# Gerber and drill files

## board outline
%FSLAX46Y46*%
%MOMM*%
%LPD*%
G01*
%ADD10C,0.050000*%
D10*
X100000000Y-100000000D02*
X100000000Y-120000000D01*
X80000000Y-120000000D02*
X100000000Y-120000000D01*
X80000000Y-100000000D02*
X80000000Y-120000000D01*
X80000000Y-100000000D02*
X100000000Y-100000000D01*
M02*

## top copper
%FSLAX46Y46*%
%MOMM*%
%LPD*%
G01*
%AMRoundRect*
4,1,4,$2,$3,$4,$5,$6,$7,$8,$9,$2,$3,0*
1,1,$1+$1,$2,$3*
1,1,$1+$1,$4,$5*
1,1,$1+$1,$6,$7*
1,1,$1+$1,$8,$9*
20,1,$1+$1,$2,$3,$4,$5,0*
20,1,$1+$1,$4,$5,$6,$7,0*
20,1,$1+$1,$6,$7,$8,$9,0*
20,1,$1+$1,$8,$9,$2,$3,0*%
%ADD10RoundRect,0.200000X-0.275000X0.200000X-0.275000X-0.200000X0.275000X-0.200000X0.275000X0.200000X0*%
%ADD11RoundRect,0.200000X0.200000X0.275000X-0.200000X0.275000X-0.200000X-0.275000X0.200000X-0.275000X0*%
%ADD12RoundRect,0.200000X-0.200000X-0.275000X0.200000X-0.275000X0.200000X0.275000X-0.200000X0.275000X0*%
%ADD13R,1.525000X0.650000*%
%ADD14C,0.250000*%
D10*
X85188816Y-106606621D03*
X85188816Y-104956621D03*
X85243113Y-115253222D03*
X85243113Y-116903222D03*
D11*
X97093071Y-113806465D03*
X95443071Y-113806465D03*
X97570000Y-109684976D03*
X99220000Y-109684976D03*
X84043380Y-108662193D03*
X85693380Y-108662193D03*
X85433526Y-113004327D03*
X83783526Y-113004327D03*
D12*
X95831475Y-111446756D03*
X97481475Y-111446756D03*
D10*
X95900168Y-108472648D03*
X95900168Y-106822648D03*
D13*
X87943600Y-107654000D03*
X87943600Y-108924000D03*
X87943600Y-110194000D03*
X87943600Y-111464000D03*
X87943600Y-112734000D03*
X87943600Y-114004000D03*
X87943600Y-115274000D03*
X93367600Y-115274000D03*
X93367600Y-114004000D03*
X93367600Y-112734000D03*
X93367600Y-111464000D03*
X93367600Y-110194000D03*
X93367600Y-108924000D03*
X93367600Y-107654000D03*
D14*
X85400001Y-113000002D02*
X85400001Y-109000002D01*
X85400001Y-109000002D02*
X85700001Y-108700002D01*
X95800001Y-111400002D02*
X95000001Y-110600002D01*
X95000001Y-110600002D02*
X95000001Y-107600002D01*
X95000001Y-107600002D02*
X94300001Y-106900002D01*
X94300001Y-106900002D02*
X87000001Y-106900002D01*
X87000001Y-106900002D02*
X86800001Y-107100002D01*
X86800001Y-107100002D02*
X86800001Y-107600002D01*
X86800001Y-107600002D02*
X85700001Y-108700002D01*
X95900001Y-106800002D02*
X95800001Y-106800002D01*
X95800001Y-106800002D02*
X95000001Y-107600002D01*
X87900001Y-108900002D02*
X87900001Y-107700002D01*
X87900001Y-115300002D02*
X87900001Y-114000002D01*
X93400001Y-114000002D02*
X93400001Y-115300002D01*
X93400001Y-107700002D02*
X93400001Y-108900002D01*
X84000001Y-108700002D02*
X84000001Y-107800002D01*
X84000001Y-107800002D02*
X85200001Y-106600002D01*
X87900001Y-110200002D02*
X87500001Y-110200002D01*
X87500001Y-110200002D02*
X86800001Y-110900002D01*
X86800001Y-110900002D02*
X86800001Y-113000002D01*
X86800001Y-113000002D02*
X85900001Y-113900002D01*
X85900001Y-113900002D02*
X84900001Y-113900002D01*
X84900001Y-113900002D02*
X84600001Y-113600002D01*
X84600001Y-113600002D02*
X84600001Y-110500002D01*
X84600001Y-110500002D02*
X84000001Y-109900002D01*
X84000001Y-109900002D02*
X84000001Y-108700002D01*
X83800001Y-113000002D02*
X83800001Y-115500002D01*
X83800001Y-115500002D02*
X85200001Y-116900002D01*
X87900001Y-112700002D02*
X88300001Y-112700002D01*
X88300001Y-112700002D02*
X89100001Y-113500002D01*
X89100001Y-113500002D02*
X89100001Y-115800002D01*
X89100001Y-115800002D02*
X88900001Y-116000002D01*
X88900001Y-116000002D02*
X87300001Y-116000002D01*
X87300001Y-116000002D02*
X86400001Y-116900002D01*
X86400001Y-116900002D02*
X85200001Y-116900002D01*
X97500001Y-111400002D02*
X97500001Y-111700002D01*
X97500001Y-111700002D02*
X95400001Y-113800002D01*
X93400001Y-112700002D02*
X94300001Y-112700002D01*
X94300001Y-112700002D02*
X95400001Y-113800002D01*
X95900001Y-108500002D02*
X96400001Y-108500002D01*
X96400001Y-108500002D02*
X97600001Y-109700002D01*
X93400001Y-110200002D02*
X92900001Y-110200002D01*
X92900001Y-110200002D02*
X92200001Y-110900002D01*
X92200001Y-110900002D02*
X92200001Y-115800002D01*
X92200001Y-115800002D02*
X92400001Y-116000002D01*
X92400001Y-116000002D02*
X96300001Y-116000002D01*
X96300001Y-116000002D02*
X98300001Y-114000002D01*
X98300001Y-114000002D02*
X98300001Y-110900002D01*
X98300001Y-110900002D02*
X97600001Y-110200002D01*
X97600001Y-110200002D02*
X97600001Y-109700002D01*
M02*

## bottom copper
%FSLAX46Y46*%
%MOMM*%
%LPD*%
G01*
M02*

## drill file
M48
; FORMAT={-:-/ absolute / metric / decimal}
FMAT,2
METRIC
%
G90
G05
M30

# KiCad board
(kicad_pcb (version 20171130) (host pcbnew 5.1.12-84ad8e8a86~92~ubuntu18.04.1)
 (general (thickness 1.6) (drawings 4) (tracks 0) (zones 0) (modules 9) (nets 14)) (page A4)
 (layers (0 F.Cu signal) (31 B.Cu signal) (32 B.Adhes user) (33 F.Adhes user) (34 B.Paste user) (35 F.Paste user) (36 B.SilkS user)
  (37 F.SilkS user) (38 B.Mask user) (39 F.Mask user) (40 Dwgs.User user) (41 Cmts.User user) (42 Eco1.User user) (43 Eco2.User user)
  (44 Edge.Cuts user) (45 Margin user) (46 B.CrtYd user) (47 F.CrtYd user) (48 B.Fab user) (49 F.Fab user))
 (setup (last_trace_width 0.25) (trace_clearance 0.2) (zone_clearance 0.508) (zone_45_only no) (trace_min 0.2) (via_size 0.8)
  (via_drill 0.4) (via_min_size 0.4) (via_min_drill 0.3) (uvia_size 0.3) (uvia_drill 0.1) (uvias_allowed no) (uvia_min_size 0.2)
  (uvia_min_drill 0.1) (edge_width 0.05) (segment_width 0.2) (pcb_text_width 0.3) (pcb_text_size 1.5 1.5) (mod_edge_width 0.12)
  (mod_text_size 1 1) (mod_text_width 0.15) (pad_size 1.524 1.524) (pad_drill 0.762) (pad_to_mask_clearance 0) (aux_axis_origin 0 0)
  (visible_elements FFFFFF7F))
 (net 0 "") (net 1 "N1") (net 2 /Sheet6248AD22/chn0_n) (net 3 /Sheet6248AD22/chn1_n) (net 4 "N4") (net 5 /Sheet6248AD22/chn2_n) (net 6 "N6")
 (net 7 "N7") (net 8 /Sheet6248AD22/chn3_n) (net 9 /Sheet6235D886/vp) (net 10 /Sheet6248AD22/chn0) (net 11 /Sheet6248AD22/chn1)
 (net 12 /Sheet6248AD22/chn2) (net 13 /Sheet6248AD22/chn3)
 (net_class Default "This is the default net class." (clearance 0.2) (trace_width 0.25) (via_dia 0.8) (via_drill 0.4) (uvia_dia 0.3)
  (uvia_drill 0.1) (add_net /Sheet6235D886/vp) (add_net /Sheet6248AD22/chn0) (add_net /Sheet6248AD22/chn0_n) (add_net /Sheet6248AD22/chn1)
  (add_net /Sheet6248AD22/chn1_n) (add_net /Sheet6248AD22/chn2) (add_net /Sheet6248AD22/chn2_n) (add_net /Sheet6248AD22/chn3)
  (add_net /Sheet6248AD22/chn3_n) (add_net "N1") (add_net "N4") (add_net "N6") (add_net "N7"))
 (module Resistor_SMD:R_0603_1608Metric (layer F.Cu) (at 85.188816 105.781621 270.000000)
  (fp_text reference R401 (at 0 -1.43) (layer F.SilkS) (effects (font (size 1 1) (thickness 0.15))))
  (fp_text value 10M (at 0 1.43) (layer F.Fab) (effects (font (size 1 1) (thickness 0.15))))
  (pad 2 smd roundrect (at 0.825 0 270.000000) (size 0.8 0.95) (layers F.Cu F.Mask F.Paste) (roundrect_rratio 0.25) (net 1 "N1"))
  (pad 1 smd roundrect (at -0.825 0 270.000000) (size 0.8 0.95) (layers F.Cu F.Mask F.Paste) (roundrect_rratio 0.25)
   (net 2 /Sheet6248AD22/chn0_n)))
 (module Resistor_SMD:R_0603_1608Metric (layer F.Cu) (at 85.243113 116.078222 270.000000)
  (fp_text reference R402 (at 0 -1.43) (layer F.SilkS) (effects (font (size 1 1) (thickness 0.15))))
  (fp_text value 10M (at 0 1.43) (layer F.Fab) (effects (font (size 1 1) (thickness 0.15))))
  (pad 1 smd roundrect (at -0.825 0 270.000000) (size 0.8 0.95) (layers F.Cu F.Mask F.Paste) (roundrect_rratio 0.25)
   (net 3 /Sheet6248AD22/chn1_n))
  (pad 2 smd roundrect (at 0.825 0 270.000000) (size 0.8 0.95) (layers F.Cu F.Mask F.Paste) (roundrect_rratio 0.25) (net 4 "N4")))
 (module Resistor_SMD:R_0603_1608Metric (layer F.Cu) (at 96.268071 113.806465 180.000000)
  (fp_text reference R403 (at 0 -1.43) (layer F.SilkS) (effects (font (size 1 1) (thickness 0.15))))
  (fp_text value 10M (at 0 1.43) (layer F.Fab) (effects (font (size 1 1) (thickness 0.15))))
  (pad 1 smd roundrect (at -0.825 0 180.000000) (size 0.8 0.95) (layers F.Cu F.Mask F.Paste) (roundrect_rratio 0.25)
   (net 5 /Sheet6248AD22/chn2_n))
  (pad 2 smd roundrect (at 0.825 0 180.000000) (size 0.8 0.95) (layers F.Cu F.Mask F.Paste) (roundrect_rratio 0.25) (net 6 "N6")))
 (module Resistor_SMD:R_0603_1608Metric (layer F.Cu) (at 98.395000 109.684976 180.000000)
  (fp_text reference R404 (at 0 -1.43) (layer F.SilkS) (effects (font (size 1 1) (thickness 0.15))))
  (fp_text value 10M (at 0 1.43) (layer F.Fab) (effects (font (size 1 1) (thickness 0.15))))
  (pad 2 smd roundrect (at 0.825 0 180.000000) (size 0.8 0.95) (layers F.Cu F.Mask F.Paste) (roundrect_rratio 0.25) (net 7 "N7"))
  (pad 1 smd roundrect (at -0.825 0 180.000000) (size 0.8 0.95) (layers F.Cu F.Mask F.Paste) (roundrect_rratio 0.25)
   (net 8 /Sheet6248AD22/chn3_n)))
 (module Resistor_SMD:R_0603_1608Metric (layer F.Cu) (at 84.868380 108.662193 180.000000)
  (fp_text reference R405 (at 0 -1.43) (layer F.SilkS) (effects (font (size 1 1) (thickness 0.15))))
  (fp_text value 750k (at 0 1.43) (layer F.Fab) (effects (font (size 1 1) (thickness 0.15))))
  (pad 2 smd roundrect (at 0.825 0 180.000000) (size 0.8 0.95) (layers F.Cu F.Mask F.Paste) (roundrect_rratio 0.25) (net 1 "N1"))
  (pad 1 smd roundrect (at -0.825 0 180.000000) (size 0.8 0.95) (layers F.Cu F.Mask F.Paste) (roundrect_rratio 0.25)
   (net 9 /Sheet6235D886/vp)))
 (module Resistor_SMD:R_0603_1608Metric (layer F.Cu) (at 84.608526 113.004327 180.000000)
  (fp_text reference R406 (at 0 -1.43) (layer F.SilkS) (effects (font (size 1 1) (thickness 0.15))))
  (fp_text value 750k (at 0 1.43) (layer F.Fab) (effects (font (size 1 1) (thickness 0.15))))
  (pad 1 smd roundrect (at -0.825 0 180.000000) (size 0.8 0.95) (layers F.Cu F.Mask F.Paste) (roundrect_rratio 0.25)
   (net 9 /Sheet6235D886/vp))
  (pad 2 smd roundrect (at 0.825 0 180.000000) (size 0.8 0.95) (layers F.Cu F.Mask F.Paste) (roundrect_rratio 0.25) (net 4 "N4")))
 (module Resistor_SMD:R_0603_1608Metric (layer F.Cu) (at 96.656475 111.446756)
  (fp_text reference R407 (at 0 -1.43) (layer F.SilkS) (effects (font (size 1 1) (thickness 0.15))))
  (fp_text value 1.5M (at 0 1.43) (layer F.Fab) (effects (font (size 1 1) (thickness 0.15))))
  (pad 1 smd roundrect (at -0.825 0) (size 0.8 0.95) (layers F.Cu F.Mask F.Paste) (roundrect_rratio 0.25) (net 9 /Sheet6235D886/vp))
  (pad 2 smd roundrect (at 0.825 0) (size 0.8 0.95) (layers F.Cu F.Mask F.Paste) (roundrect_rratio 0.25) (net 6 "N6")))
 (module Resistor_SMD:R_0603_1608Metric (layer F.Cu) (at 95.900168 107.647648 270.000000)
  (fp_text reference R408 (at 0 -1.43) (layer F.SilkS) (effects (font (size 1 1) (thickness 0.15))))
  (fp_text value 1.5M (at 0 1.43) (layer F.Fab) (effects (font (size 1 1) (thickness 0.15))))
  (pad 2 smd roundrect (at 0.825 0 270.000000) (size 0.8 0.95) (layers F.Cu F.Mask F.Paste) (roundrect_rratio 0.25) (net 7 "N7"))
  (pad 1 smd roundrect (at -0.825 0 270.000000) (size 0.8 0.95) (layers F.Cu F.Mask F.Paste) (roundrect_rratio 0.25)
   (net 9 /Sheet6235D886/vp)))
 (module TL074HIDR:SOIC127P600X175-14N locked (layer F.Cu) (at 90.655600 111.464000)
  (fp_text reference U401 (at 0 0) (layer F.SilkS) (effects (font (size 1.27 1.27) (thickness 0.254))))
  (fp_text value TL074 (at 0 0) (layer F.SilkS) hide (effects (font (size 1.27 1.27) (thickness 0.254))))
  (pad 1 smd rect (at -2.712 -3.81 90.000000) (size 0.65 1.525) (layers F.Cu F.Mask F.Paste) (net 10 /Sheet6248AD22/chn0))
  (pad 2 smd rect (at -2.712 -2.54 90.000000) (size 0.65 1.525) (layers F.Cu F.Mask F.Paste) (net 10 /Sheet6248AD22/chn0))
  (pad 3 smd rect (at -2.712 -1.27 90.000000) (size 0.65 1.525) (layers F.Cu F.Mask F.Paste) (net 1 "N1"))
  (pad 4 smd rect (at -2.712 0 90.000000) (size 0.65 1.525) (layers F.Cu F.Mask F.Paste))
  (pad 5 smd rect (at -2.712 1.27 90.000000) (size 0.65 1.525) (layers F.Cu F.Mask F.Paste) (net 4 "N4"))
  (pad 6 smd rect (at -2.712 2.54 90.000000) (size 0.65 1.525) (layers F.Cu F.Mask F.Paste) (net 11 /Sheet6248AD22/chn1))
  (pad 7 smd rect (at -2.712 3.81 90.000000) (size 0.65 1.525) (layers F.Cu F.Mask F.Paste) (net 11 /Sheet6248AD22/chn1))
  (pad 8 smd rect (at 2.712 3.81 90.000000) (size 0.65 1.525) (layers F.Cu F.Mask F.Paste) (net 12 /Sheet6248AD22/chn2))
  (pad 9 smd rect (at 2.712 2.54 90.000000) (size 0.65 1.525) (layers F.Cu F.Mask F.Paste) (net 12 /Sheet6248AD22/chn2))
  (pad 10 smd rect (at 2.712 1.27 90.000000) (size 0.65 1.525) (layers F.Cu F.Mask F.Paste) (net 6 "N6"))
  (pad 11 smd rect (at 2.712 0 90.000000) (size 0.65 1.525) (layers F.Cu F.Mask F.Paste))
  (pad 12 smd rect (at 2.712 -1.27 90.000000) (size 0.65 1.525) (layers F.Cu F.Mask F.Paste) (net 7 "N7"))
  (pad 13 smd rect (at 2.712 -2.54 90.000000) (size 0.65 1.525) (layers F.Cu F.Mask F.Paste) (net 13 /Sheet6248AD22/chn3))
  (pad 14 smd rect (at 2.712 -3.81 90.000000) (size 0.65 1.525) (layers F.Cu F.Mask F.Paste) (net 13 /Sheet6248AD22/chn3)))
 (gr_line (start 100 100) (end 100 120) (layer Edge.Cuts) (width 0.05))
 (gr_line (start 80 120) (end 100 120) (layer Edge.Cuts) (width 0.05))
 (gr_line (start 80 100) (end 80 120) (layer Edge.Cuts) (width 0.05))
 (gr_line (start 80 100) (end 100 100) (layer Edge.Cuts) (width 0.05))
 (segment (start 85.400001 113.000002) (end 85.400001 109.000002) (width 0.250000) (layer F.Cu) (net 9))
 (segment (start 85.400001 109.000002) (end 85.700001 108.700002) (width 0.250000) (layer F.Cu) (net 9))
 (segment (start 95.800001 111.400002) (end 95.000001 110.600002) (width 0.250000) (layer F.Cu) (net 9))
 (segment (start 95.000001 110.600002) (end 95.000001 107.600002) (width 0.250000) (layer F.Cu) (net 9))
 (segment (start 95.000001 107.600002) (end 94.300001 106.900002) (width 0.250000) (layer F.Cu) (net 9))
 (segment (start 94.300001 106.900002) (end 87.000001 106.900002) (width 0.250000) (layer F.Cu) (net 9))
 (segment (start 87.000001 106.900002) (end 86.800001 107.100002) (width 0.250000) (layer F.Cu) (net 9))
 (segment (start 86.800001 107.100002) (end 86.800001 107.600002) (width 0.250000) (layer F.Cu) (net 9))
 (segment (start 86.800001 107.600002) (end 85.700001 108.700002) (width 0.250000) (layer F.Cu) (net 9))
 (segment (start 95.900001 106.800002) (end 95.800001 106.800002) (width 0.250000) (layer F.Cu) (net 9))
 (segment (start 95.800001 106.800002) (end 95.000001 107.600002) (width 0.250000) (layer F.Cu) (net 9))
 (segment (start 87.900001 108.900002) (end 87.900001 107.700002) (width 0.250000) (layer F.Cu) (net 10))
 (segment (start 87.900001 115.300002) (end 87.900001 114.000002) (width 0.250000) (layer F.Cu) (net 11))
 (segment (start 93.400001 114.000002) (end 93.400001 115.300002) (width 0.250000) (layer F.Cu) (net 12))
 (segment (start 93.400001 107.700002) (end 93.400001 108.900002) (width 0.250000) (layer F.Cu) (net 13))
 (segment (start 84.000001 108.700002) (end 84.000001 107.800002) (width 0.250000) (layer F.Cu) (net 1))
 (segment (start 84.000001 107.800002) (end 85.200001 106.600002) (width 0.250000) (layer F.Cu) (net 1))
 (segment (start 87.900001 110.200002) (end 87.500001 110.200002) (width 0.250000) (layer F.Cu) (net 1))
 (segment (start 87.500001 110.200002) (end 86.800001 110.900002) (width 0.250000) (layer F.Cu) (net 1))
 (segment (start 86.800001 110.900002) (end 86.800001 113.000002) (width 0.250000) (layer F.Cu) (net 1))
 (segment (start 86.800001 113.000002) (end 85.900001 113.900002) (width 0.250000) (layer F.Cu) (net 1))
 (segment (start 85.900001 113.900002) (end 84.900001 113.900002) (width 0.250000) (layer F.Cu) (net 1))
 (segment (start 84.900001 113.900002) (end 84.600001 113.600002) (width 0.250000) (layer F.Cu) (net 1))
 (segment (start 84.600001 113.600002) (end 84.600001 110.500002) (width 0.250000) (layer F.Cu) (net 1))
 (segment (start 84.600001 110.500002) (end 84.000001 109.900002) (width 0.250000) (layer F.Cu) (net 1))
 (segment (start 84.000001 109.900002) (end 84.000001 108.700002) (width 0.250000) (layer F.Cu) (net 1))
 (segment (start 83.800001 113.000002) (end 83.800001 115.500002) (width 0.250000) (layer F.Cu) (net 4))
 (segment (start 83.800001 115.500002) (end 85.200001 116.900002) (width 0.250000) (layer F.Cu) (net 4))
 (segment (start 87.900001 112.700002) (end 88.300001 112.700002) (width 0.250000) (layer F.Cu) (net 4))
 (segment (start 88.300001 112.700002) (end 89.100001 113.500002) (width 0.250000) (layer F.Cu) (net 4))
 (segment (start 89.100001 113.500002) (end 89.100001 115.800002) (width 0.250000) (layer F.Cu) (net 4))
 (segment (start 89.100001 115.800002) (end 88.900001 116.000002) (width 0.250000) (layer F.Cu) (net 4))
 (segment (start 88.900001 116.000002) (end 87.300001 116.000002) (width 0.250000) (layer F.Cu) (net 4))
 (segment (start 87.300001 116.000002) (end 86.400001 116.900002) (width 0.250000) (layer F.Cu) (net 4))
 (segment (start 86.400001 116.900002) (end 85.200001 116.900002) (width 0.250000) (layer F.Cu) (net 4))
 (segment (start 97.500001 111.400002) (end 97.500001 111.700002) (width 0.250000) (layer F.Cu) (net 6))
 (segment (start 97.500001 111.700002) (end 95.400001 113.800002) (width 0.250000) (layer F.Cu) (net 6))
 (segment (start 93.400001 112.700002) (end 94.300001 112.700002) (width 0.250000) (layer F.Cu) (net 6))
 (segment (start 94.300001 112.700002) (end 95.400001 113.800002) (width 0.250000) (layer F.Cu) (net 6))
 (segment (start 95.900001 108.500002) (end 96.400001 108.500002) (width 0.250000) (layer F.Cu) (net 7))
 (segment (start 96.400001 108.500002) (end 97.600001 109.700002) (width 0.250000) (layer F.Cu) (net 7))
 (segment (start 93.400001 110.200002) (end 92.900001 110.200002) (width 0.250000) (layer F.Cu) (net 7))
 (segment (start 92.900001 110.200002) (end 92.200001 110.900002) (width 0.250000) (layer F.Cu) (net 7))
 (segment (start 92.200001 110.900002) (end 92.200001 115.800002) (width 0.250000) (layer F.Cu) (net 7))
 (segment (start 92.200001 115.800002) (end 92.400001 116.000002) (width 0.250000) (layer F.Cu) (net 7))
 (segment (start 92.400001 116.000002) (end 96.300001 116.000002) (width 0.250000) (layer F.Cu) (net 7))
 (segment (start 96.300001 116.000002) (end 98.300001 114.000002) (width 0.250000) (layer F.Cu) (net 7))
 (segment (start 98.300001 114.000002) (end 98.300001 110.900002) (width 0.250000) (layer F.Cu) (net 7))
 (segment (start 98.300001 110.900002) (end 97.600001 110.200002) (width 0.250000) (layer F.Cu) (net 7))
 (segment (start 97.600001 110.200002) (end 97.600001 109.700002) (width 0.250000) (layer F.Cu) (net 7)))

